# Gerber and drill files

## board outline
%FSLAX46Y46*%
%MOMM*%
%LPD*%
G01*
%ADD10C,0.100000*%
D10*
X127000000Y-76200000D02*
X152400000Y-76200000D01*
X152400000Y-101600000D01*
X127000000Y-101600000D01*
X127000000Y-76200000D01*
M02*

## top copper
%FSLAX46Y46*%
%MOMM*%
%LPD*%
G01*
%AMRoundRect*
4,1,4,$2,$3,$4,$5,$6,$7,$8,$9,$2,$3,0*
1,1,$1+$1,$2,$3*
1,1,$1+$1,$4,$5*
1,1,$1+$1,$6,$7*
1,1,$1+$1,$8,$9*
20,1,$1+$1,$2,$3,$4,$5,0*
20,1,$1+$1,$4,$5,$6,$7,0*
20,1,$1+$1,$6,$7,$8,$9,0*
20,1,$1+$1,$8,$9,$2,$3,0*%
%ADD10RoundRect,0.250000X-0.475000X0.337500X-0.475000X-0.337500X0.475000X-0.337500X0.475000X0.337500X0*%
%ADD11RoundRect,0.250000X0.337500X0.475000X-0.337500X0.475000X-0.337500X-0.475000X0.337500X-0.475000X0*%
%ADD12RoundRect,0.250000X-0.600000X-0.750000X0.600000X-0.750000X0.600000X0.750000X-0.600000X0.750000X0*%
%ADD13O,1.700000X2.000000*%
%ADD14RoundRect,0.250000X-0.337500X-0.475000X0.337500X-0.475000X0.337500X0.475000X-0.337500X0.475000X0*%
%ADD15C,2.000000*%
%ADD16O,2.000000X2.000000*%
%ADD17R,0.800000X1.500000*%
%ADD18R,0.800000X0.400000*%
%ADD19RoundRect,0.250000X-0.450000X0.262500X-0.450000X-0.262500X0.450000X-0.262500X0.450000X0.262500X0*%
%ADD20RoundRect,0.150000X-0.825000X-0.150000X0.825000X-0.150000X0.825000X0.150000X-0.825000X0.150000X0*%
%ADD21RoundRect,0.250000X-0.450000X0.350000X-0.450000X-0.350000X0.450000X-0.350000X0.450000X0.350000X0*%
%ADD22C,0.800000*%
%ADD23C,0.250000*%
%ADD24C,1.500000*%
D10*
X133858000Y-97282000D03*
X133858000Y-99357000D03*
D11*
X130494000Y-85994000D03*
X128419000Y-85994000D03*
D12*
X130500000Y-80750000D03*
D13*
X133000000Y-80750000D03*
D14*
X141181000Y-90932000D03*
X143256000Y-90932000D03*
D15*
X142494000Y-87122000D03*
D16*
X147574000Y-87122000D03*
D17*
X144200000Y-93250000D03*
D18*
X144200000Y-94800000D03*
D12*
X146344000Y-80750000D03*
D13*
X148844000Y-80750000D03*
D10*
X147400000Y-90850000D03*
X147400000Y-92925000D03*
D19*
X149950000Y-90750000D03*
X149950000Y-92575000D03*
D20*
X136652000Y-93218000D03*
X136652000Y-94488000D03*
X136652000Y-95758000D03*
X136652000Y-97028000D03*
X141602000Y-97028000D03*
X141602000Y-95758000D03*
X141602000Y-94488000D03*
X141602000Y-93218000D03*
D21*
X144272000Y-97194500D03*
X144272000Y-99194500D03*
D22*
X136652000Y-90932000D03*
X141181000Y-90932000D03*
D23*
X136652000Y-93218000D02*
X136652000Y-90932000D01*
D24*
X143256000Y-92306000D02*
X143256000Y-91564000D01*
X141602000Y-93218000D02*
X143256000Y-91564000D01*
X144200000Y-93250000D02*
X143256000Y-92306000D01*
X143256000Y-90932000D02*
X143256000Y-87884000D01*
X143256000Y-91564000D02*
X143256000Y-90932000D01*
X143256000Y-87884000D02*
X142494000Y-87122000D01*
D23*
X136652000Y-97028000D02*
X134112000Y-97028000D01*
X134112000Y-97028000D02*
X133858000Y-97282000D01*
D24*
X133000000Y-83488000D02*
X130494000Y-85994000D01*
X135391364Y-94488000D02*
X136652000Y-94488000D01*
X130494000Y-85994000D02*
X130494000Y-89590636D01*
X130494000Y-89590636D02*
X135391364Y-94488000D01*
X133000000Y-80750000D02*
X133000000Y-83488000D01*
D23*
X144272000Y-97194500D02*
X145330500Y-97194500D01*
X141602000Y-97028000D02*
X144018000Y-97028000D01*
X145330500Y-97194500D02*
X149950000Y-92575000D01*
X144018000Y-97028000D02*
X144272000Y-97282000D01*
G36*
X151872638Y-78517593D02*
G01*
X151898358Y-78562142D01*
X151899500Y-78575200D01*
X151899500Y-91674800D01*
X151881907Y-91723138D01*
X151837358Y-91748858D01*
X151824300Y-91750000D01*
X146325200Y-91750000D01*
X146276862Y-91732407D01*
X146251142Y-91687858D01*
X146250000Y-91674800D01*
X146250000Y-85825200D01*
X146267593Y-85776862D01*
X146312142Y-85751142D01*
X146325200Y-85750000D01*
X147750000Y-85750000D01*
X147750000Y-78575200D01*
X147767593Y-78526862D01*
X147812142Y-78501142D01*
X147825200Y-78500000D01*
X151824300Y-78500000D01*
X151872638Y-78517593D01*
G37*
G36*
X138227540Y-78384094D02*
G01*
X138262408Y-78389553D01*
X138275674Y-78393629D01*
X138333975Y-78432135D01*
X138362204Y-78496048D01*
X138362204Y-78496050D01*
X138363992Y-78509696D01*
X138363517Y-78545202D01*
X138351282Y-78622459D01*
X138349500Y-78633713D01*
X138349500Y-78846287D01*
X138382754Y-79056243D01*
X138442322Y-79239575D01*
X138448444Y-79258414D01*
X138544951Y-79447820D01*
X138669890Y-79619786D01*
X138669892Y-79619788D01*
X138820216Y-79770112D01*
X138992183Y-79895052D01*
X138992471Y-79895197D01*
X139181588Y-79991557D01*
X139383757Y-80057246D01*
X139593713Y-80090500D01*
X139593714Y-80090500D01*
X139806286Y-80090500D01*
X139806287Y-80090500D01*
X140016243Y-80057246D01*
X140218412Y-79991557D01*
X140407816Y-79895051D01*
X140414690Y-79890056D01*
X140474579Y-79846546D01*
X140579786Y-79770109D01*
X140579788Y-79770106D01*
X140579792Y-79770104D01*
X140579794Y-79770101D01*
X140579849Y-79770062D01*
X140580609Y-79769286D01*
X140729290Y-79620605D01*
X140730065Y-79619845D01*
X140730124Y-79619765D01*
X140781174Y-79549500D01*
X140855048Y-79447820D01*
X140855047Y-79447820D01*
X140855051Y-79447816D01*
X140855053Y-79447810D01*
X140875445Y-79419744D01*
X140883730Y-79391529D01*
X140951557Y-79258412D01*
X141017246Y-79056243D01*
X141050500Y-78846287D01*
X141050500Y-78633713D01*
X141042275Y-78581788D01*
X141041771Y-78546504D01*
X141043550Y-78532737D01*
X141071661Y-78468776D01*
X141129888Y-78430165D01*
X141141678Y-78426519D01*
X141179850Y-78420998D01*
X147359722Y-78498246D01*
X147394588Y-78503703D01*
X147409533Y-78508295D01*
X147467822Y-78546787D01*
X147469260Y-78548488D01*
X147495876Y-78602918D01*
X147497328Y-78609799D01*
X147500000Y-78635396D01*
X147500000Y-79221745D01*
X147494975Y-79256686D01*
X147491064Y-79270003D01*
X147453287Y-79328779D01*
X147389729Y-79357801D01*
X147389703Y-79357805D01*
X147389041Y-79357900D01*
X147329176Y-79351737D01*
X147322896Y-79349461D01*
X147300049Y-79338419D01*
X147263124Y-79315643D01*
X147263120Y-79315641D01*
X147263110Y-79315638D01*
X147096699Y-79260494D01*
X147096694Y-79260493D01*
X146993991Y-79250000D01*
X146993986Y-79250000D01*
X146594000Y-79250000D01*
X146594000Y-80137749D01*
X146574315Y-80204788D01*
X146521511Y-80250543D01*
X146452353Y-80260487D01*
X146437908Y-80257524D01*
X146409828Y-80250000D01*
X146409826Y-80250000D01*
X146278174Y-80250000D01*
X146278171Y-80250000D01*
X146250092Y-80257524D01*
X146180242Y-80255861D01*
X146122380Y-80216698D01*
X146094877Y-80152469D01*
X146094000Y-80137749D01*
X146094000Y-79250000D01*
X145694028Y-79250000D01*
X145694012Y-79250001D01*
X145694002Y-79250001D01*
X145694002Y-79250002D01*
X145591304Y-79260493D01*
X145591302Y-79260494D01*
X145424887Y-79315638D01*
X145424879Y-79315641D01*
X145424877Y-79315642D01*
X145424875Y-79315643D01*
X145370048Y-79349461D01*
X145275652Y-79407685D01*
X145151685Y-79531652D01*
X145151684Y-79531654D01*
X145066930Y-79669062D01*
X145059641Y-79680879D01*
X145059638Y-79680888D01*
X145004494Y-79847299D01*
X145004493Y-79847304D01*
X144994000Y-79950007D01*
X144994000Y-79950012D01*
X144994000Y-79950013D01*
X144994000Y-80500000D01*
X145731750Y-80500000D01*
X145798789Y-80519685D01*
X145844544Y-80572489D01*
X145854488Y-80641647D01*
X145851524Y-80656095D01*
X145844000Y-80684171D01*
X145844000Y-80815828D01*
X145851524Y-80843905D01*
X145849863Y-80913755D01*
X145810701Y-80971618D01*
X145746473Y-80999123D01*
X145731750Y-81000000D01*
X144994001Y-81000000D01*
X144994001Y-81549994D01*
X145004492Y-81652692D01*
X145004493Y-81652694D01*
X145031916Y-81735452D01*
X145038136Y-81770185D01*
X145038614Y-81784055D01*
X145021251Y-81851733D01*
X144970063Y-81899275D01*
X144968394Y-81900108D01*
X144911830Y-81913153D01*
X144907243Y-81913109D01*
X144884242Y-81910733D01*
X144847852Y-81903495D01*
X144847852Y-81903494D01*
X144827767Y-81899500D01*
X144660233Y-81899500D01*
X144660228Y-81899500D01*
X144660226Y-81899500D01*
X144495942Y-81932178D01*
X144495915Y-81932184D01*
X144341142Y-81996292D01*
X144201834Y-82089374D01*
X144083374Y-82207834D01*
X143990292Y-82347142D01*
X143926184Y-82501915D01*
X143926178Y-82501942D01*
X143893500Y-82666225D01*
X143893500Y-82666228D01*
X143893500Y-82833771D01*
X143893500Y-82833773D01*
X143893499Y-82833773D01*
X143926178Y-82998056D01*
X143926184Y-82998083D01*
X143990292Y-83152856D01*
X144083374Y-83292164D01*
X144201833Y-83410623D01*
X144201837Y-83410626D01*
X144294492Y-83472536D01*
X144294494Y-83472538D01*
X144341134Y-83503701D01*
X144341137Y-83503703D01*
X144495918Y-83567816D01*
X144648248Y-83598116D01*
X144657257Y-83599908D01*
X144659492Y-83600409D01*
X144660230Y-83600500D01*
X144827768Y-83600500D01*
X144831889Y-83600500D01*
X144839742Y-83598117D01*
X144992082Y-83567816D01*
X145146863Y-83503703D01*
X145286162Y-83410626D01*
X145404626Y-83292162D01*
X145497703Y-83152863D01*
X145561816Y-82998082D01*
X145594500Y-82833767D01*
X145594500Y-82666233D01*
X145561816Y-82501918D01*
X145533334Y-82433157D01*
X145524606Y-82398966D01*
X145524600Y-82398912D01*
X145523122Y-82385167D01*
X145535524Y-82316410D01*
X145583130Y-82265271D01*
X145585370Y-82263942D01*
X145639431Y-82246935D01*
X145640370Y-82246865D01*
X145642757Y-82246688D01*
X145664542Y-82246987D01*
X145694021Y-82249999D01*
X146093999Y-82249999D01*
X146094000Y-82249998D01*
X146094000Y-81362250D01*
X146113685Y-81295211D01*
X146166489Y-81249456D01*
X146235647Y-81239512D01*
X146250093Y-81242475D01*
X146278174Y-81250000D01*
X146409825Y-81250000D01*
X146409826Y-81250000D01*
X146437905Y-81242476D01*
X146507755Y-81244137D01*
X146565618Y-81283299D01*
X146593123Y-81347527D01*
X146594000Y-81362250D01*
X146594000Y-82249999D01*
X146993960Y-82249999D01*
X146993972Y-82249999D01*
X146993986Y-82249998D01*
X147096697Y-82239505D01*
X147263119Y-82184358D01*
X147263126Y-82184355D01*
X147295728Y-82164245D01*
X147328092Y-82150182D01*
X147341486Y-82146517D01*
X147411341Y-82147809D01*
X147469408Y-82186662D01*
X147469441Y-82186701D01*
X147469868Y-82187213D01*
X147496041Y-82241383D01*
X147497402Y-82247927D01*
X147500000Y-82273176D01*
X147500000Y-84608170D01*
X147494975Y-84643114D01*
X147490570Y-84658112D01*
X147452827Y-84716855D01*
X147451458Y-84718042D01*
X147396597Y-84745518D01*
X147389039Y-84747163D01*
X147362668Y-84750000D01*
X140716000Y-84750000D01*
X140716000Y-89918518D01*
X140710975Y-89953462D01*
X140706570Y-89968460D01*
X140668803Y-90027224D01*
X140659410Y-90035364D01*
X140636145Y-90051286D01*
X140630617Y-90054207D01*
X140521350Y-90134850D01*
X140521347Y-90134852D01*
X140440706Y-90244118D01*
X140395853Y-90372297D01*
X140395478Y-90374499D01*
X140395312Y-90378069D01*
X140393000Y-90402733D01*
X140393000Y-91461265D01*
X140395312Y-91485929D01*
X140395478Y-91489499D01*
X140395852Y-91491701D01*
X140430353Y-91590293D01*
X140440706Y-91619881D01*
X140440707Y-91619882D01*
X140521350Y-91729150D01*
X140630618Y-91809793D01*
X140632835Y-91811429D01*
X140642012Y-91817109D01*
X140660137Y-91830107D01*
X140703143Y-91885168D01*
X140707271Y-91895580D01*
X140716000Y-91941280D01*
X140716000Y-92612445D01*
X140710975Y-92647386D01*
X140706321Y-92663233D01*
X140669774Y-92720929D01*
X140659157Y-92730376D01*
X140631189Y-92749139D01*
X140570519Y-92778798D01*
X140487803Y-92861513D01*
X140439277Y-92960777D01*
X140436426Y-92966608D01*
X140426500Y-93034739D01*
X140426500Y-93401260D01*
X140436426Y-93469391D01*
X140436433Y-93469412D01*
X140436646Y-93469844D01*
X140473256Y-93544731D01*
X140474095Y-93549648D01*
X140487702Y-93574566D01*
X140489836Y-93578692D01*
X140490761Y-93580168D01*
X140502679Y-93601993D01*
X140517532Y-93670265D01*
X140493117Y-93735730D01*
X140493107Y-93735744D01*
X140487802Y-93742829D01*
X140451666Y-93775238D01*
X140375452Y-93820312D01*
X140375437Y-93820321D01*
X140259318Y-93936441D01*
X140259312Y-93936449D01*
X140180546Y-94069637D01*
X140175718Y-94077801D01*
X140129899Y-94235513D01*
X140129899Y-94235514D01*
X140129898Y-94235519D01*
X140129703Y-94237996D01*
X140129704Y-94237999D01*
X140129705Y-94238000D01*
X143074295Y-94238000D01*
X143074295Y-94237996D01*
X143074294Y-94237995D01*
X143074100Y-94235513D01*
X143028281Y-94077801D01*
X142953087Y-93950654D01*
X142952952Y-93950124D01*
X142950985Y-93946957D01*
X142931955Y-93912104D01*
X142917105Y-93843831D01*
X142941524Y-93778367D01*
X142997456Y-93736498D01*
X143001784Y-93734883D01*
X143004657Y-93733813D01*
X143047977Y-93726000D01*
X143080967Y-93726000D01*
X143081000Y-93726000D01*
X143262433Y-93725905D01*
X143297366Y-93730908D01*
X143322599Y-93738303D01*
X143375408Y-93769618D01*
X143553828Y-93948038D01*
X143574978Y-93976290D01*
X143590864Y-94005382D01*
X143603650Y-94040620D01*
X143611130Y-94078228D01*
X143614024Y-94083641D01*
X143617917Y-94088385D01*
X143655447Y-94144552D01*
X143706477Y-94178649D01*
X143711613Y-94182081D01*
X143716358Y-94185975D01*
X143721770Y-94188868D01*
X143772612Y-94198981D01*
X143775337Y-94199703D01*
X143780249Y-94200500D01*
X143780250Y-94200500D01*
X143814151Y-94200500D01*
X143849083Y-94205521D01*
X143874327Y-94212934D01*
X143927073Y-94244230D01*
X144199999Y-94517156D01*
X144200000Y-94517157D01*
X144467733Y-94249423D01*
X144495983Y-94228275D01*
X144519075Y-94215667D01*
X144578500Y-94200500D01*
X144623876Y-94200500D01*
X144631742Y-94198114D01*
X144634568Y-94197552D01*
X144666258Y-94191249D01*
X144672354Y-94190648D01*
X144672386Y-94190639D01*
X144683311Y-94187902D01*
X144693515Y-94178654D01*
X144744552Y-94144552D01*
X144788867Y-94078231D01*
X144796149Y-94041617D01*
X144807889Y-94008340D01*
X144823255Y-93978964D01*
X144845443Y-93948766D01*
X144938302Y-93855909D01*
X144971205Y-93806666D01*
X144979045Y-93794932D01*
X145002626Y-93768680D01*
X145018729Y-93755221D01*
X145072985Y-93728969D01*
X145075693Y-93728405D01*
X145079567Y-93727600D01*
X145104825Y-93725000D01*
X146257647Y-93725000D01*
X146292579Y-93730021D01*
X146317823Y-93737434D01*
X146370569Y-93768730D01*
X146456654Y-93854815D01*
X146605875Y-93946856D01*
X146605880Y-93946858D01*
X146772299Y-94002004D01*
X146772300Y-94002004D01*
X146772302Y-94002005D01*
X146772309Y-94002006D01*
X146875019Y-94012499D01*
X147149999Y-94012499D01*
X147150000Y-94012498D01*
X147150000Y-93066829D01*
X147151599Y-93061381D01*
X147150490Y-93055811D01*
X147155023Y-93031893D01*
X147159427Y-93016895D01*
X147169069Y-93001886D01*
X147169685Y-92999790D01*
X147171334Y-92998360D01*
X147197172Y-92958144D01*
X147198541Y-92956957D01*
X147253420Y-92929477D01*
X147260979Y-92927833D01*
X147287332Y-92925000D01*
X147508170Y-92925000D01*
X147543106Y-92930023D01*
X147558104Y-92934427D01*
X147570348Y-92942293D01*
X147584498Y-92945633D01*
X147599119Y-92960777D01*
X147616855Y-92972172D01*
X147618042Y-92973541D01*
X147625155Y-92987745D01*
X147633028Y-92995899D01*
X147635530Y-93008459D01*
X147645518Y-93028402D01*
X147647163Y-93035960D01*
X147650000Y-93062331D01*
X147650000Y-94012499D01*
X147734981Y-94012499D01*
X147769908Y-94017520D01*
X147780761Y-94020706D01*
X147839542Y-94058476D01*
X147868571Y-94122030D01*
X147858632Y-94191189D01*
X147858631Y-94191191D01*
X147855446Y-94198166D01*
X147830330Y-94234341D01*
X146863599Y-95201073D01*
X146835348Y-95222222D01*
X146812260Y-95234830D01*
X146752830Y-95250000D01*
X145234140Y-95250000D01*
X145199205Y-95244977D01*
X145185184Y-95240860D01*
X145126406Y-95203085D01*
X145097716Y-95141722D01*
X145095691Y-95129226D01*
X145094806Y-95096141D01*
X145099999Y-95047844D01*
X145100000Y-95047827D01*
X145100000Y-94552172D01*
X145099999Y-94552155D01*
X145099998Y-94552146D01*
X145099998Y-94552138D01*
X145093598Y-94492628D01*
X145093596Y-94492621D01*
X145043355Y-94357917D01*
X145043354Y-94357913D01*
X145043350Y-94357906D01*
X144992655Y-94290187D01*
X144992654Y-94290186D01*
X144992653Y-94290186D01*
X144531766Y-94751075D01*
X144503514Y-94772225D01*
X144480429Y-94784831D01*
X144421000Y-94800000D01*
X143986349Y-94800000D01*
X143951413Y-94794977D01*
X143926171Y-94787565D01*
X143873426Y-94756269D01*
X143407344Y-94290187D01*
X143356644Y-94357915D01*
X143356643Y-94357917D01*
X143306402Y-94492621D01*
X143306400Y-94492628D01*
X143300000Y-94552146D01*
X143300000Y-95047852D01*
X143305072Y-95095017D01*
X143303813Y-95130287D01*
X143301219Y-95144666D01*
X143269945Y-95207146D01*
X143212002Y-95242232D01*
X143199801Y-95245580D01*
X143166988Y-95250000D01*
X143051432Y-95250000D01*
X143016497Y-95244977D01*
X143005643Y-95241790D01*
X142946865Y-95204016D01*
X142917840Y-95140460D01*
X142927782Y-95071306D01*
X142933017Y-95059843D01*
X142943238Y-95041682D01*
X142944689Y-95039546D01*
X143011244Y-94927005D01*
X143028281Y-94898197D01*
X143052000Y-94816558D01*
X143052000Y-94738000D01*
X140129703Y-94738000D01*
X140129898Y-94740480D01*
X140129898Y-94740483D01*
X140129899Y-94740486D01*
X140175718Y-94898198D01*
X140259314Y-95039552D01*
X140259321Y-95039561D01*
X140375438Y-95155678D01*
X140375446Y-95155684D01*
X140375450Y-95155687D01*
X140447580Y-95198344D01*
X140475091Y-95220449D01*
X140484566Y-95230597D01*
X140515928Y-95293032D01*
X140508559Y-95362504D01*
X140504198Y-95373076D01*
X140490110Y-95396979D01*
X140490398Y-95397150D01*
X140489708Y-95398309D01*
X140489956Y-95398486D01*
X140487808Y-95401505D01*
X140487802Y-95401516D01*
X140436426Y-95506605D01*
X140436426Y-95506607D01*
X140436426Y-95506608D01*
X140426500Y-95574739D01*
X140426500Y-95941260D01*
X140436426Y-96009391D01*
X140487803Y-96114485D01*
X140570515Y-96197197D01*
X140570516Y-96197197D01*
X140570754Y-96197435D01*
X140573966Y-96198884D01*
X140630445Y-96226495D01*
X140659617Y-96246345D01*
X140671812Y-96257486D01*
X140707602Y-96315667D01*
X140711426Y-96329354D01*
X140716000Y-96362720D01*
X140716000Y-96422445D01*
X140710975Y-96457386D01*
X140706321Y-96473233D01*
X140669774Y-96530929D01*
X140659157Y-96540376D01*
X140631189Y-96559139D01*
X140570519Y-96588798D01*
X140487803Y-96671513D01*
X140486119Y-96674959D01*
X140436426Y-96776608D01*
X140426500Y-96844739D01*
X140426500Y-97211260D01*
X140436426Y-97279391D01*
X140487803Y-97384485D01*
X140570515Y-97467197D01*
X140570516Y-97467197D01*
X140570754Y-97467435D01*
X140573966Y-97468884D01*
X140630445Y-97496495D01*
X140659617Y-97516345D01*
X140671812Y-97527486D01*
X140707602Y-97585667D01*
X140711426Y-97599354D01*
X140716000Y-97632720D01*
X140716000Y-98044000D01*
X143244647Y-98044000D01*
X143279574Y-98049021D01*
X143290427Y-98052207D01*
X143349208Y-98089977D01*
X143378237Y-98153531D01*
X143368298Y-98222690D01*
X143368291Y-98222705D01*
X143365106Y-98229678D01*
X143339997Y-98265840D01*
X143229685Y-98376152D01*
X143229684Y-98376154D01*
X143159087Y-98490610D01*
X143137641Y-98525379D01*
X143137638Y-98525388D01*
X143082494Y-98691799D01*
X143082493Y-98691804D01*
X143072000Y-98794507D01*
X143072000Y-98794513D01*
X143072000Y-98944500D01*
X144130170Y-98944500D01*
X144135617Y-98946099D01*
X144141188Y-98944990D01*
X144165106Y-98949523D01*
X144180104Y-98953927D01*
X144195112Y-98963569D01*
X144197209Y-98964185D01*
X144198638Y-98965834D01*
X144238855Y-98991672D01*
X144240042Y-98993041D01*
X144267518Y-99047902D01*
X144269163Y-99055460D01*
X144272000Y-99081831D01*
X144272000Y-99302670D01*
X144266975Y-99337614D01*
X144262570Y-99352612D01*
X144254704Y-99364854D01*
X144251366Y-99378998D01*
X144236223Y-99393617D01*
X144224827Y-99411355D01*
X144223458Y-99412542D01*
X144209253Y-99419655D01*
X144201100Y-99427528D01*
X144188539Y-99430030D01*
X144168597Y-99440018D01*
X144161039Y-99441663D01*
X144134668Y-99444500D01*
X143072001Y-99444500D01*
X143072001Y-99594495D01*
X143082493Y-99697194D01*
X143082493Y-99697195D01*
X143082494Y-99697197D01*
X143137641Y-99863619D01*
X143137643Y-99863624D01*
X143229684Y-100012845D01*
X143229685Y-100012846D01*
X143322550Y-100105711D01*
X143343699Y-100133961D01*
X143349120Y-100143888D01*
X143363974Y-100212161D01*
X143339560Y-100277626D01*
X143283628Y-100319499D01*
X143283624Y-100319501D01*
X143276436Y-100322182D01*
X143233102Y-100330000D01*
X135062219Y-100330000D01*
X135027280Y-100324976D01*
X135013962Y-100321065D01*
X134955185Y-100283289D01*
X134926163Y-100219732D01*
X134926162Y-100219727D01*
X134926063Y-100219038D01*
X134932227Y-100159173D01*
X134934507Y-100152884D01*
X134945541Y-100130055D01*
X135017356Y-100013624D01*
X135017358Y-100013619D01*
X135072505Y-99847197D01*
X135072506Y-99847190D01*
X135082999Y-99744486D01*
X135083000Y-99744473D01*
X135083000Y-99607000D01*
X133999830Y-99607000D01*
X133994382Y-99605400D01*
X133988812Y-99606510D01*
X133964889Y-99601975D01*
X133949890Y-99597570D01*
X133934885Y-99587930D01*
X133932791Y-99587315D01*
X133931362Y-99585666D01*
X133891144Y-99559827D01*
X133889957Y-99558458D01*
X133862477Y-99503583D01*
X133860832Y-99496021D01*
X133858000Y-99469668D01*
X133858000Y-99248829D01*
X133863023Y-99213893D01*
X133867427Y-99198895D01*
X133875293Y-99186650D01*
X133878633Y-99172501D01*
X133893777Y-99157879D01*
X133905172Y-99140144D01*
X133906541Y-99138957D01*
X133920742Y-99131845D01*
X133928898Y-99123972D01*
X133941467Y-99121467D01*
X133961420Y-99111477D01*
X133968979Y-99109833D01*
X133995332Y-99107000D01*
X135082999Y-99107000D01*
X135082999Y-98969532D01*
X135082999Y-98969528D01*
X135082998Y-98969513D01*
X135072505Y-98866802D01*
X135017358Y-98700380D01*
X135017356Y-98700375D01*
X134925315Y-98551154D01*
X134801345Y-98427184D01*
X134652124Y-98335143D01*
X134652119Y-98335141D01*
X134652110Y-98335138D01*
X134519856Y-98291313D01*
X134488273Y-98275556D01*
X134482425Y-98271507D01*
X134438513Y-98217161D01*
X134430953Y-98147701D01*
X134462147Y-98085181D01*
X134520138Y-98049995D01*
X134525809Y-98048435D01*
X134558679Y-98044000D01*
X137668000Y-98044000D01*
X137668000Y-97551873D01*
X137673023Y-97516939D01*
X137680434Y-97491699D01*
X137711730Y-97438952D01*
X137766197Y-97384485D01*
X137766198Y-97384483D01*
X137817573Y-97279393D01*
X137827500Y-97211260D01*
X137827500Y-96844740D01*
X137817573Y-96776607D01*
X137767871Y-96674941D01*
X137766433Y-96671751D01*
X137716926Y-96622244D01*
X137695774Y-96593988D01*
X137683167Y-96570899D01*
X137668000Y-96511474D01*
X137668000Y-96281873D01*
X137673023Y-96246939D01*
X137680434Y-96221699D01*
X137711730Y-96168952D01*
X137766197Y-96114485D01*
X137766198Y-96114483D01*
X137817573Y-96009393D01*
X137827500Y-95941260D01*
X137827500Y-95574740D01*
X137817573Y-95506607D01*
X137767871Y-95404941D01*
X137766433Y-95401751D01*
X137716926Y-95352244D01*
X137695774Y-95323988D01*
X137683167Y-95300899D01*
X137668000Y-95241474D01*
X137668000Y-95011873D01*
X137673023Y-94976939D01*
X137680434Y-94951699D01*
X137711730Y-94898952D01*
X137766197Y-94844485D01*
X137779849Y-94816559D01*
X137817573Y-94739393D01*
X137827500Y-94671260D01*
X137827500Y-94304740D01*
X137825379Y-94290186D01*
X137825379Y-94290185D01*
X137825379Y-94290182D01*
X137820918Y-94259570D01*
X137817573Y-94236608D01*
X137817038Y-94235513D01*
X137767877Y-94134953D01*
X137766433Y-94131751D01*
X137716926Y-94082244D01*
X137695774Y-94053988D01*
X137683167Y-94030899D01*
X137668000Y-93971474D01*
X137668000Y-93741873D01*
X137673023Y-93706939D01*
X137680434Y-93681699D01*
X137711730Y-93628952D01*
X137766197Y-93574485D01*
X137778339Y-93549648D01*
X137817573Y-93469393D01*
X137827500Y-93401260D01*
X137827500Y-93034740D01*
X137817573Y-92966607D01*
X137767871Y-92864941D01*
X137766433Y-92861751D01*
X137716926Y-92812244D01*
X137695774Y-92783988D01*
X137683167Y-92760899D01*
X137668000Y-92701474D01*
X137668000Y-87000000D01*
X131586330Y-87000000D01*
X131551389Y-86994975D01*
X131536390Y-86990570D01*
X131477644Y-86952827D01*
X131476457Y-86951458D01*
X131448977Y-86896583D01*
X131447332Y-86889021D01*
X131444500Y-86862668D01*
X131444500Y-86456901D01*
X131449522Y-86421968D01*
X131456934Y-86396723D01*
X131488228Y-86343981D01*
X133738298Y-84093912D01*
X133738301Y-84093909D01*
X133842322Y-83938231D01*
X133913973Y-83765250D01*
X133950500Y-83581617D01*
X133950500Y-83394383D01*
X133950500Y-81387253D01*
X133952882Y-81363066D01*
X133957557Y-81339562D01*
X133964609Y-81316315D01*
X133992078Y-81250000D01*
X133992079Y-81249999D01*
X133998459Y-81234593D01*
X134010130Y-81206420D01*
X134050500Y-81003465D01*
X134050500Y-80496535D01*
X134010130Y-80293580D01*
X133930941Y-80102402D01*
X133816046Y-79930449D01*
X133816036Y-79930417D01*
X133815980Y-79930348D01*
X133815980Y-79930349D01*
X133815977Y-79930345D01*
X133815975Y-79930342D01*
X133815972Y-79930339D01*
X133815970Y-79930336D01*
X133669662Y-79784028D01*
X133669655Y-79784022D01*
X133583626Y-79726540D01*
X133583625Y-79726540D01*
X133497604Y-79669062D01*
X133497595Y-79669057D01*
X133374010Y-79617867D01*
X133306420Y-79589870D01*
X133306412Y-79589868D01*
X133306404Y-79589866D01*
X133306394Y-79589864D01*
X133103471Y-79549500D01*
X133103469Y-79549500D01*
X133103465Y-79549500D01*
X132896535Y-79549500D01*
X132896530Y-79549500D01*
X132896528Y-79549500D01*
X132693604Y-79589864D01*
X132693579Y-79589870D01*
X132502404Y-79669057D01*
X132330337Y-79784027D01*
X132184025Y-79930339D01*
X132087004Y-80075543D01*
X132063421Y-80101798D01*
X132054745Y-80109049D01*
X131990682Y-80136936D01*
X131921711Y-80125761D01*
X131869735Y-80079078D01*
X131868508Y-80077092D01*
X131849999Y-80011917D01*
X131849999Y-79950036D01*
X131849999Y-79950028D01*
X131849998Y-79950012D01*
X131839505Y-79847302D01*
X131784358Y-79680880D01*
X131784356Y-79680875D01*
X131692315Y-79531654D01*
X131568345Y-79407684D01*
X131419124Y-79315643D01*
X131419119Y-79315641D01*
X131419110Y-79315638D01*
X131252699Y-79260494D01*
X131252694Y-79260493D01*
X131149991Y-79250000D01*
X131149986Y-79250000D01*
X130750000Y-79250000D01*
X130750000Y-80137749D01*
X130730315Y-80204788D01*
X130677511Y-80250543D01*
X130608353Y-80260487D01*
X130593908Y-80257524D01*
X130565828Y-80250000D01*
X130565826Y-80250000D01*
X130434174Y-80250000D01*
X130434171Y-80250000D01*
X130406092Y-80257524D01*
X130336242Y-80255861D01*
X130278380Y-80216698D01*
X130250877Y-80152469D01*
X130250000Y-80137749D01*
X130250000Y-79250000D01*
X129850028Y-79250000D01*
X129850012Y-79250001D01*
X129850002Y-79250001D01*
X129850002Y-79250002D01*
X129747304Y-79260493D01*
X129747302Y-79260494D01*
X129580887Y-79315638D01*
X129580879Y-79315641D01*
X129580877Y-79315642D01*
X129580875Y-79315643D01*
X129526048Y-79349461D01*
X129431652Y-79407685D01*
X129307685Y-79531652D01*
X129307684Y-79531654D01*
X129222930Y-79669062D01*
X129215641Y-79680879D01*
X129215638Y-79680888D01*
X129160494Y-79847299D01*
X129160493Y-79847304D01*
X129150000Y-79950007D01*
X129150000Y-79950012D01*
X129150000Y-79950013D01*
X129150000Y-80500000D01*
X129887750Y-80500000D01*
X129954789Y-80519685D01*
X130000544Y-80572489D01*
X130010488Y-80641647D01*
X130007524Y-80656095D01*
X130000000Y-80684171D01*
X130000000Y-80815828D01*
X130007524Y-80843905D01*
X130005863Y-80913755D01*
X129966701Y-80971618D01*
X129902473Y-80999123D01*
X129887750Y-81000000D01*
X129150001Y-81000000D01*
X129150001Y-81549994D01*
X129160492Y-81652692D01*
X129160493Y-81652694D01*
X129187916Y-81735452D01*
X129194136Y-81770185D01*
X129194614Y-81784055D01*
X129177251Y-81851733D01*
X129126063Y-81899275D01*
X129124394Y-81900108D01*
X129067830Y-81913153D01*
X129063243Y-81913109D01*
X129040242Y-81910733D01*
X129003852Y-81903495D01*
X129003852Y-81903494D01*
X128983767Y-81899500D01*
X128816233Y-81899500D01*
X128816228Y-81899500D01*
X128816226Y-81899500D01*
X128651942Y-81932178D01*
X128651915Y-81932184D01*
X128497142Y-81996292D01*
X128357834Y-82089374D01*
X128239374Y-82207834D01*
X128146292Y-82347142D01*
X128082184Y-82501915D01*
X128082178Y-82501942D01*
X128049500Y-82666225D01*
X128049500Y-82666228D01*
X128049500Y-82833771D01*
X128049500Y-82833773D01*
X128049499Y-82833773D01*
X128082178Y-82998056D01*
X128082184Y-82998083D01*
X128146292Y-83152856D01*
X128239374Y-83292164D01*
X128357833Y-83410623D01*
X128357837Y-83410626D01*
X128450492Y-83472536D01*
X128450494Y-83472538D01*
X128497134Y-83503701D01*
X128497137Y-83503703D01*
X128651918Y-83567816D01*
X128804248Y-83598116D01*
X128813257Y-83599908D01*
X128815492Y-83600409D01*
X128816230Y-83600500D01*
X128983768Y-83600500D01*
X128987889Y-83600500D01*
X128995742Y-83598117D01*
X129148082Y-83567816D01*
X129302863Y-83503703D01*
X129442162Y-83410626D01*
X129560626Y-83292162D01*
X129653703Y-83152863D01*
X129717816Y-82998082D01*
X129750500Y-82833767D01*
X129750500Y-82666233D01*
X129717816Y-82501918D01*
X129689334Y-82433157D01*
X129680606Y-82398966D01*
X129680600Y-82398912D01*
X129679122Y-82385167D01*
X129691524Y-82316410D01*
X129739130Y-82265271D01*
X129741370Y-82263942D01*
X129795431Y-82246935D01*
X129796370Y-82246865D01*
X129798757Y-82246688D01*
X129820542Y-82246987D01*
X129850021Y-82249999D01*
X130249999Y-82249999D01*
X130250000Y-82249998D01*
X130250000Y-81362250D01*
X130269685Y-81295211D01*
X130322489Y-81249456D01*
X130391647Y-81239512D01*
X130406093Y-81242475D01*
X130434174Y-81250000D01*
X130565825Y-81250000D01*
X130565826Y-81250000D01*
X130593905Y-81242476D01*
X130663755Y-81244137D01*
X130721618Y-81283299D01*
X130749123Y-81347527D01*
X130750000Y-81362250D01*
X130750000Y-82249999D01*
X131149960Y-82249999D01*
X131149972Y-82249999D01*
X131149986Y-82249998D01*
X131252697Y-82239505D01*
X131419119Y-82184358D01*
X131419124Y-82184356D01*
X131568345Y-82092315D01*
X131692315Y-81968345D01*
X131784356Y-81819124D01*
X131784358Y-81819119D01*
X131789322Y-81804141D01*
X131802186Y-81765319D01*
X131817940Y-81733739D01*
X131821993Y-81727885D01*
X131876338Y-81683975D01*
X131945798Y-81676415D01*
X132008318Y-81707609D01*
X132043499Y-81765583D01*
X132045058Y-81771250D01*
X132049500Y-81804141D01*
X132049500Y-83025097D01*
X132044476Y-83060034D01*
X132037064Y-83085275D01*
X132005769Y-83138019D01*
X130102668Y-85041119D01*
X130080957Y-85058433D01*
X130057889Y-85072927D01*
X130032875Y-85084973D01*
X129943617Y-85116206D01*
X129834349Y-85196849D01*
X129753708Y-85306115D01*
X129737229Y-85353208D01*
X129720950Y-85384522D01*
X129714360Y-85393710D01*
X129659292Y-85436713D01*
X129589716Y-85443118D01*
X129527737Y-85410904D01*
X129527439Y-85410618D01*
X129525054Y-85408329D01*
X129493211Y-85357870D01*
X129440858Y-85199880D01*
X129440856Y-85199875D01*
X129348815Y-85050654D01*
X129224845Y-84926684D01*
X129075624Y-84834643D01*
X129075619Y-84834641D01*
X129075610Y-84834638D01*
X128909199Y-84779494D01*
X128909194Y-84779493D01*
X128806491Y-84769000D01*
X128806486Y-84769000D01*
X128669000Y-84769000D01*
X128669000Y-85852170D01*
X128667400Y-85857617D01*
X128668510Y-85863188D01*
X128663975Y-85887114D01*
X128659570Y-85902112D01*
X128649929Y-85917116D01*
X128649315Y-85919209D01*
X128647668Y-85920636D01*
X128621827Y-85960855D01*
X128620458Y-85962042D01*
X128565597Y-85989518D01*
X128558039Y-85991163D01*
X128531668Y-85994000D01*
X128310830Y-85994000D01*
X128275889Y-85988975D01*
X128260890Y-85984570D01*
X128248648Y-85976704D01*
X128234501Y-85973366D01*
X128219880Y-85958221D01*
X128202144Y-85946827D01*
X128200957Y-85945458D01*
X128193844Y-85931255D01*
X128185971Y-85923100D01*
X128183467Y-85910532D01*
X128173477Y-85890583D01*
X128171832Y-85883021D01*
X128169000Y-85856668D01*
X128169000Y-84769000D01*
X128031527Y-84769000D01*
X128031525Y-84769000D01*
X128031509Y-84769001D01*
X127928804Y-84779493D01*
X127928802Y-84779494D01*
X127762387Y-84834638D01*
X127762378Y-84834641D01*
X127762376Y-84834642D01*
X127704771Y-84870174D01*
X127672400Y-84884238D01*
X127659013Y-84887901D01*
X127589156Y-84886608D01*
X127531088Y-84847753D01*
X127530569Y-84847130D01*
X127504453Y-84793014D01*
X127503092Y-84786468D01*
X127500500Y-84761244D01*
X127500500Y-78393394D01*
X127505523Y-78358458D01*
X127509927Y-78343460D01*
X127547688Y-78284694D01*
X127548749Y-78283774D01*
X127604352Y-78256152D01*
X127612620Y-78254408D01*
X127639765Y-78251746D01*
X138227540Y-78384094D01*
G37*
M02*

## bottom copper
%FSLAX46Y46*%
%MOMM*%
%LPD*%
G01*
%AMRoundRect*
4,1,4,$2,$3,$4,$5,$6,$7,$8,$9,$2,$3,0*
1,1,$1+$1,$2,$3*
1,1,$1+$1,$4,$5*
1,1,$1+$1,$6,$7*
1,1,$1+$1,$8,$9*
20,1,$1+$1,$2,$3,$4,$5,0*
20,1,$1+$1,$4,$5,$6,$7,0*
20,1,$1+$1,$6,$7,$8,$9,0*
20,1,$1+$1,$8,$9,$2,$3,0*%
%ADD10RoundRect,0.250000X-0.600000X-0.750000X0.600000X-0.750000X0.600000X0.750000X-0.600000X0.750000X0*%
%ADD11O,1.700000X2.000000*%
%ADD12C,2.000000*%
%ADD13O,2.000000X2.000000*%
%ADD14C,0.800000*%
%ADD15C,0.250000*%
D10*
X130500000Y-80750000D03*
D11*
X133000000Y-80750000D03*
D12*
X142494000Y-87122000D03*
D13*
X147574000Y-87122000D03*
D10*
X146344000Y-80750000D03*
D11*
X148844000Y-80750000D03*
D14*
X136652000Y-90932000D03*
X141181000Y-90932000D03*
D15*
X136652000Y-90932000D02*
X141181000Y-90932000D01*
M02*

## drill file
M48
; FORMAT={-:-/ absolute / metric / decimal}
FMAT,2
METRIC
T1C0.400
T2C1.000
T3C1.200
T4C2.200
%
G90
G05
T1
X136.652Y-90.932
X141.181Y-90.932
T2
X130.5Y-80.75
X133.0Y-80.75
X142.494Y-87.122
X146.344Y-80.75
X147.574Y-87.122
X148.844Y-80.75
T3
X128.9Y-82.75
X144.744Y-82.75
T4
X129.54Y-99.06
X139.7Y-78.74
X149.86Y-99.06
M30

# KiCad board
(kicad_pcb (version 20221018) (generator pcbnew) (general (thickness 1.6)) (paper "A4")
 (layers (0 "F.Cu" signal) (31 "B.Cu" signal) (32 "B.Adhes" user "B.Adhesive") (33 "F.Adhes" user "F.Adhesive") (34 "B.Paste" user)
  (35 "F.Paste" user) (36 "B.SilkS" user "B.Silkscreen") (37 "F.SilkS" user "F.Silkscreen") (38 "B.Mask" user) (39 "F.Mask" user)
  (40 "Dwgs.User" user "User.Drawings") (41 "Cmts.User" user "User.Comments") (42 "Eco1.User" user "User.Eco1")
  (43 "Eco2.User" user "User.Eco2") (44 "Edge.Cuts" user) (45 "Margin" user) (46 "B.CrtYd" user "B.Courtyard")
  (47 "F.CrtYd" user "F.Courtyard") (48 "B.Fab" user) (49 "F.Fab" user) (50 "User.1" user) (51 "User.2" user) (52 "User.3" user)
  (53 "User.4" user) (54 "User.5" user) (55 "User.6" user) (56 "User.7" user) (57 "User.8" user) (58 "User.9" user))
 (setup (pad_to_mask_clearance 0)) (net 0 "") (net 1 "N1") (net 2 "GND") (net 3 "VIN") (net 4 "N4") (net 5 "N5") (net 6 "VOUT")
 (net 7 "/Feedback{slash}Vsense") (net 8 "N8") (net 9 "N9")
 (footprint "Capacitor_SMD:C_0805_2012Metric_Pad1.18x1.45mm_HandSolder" (layer "F.Cu") (at 133.858 98.3195 -90)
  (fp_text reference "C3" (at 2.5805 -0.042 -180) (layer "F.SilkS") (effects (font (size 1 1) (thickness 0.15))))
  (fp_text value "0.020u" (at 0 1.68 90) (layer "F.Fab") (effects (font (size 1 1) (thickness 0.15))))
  (pad "1" smd roundrect (at -1.0375 0 270) (size 1.175 1.45) (layers "F.Cu" "F.Paste" "F.Mask") (roundrect_rratio 0.212766) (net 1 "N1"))
  (pad "2" smd roundrect (at 1.0375 0 270) (size 1.175 1.45) (layers "F.Cu" "F.Paste" "F.Mask") (roundrect_rratio 0.212766) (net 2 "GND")))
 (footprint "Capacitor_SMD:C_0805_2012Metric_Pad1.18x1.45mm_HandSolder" (layer "F.Cu") (at 129.4565 85.994 180)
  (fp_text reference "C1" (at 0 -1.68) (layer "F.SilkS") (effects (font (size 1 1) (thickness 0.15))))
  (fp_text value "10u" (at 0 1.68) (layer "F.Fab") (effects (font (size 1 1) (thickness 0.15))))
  (pad "1" smd roundrect (at -1.0375 0 180) (size 1.175 1.45) (layers "F.Cu" "F.Paste" "F.Mask") (roundrect_rratio 0.212766) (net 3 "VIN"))
  (pad "2" smd roundrect (at 1.0375 0 180) (size 1.175 1.45) (layers "F.Cu" "F.Paste" "F.Mask") (roundrect_rratio 0.212766) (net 2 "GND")))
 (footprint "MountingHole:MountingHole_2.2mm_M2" (layer "F.Cu") (at 139.7 78.74)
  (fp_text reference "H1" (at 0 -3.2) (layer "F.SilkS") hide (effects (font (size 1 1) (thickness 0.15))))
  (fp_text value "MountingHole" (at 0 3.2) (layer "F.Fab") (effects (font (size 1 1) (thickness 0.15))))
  (pad "" np_thru_hole circle (at 0 0) (size 2.2 2.2) (drill 2.2) (layers "*.Cu" "*.Mask")))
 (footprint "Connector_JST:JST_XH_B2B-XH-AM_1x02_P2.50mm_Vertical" (layer "F.Cu") (at 130.5 80.75)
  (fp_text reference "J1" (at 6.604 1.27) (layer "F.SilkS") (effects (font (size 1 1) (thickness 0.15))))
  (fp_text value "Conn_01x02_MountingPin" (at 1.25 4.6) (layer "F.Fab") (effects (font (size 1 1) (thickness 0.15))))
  (pad "" np_thru_hole circle (at -1.6 2) (size 1.2 1.2) (drill 1.2) (layers "*.Cu" "*.Mask"))
  (pad "1" thru_hole roundrect (at 0 0) (size 1.7 2) (drill 1) (layers "*.Cu" "*.Mask") (roundrect_rratio 0.147059) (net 2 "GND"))
  (pad "2" thru_hole oval (at 2.5 0) (size 1.7 2) (drill 1) (layers "*.Cu" "*.Mask") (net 3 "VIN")))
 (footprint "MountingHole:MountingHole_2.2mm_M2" (layer "F.Cu") (at 129.54 99.06)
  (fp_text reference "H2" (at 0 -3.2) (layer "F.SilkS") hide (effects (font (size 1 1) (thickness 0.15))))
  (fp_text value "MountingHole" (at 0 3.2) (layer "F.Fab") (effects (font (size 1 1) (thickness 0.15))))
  (pad "" np_thru_hole circle (at 0 0) (size 2.2 2.2) (drill 2.2) (layers "*.Cu" "*.Mask")))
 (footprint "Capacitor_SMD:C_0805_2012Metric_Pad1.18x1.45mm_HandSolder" (layer "F.Cu") (at 142.2185 90.932)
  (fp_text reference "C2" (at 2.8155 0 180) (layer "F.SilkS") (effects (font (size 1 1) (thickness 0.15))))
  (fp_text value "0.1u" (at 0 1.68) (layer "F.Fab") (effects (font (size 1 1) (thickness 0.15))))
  (pad "1" smd roundrect (at -1.0375 0) (size 1.175 1.45) (layers "F.Cu" "F.Paste" "F.Mask") (roundrect_rratio 0.212766) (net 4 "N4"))
  (pad "2" smd roundrect (at 1.0375 0) (size 1.175 1.45) (layers "F.Cu" "F.Paste" "F.Mask") (roundrect_rratio 0.212766) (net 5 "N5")))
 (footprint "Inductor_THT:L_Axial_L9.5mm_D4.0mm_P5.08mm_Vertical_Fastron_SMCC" (layer "F.Cu") (at 142.494 87.122)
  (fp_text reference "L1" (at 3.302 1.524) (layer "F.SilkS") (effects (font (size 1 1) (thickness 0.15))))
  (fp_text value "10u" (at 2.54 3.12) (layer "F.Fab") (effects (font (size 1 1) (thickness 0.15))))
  (pad "1" thru_hole circle (at 0 0) (size 2 2) (drill 1) (layers "*.Cu" "*.Mask") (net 5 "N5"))
  (pad "2" thru_hole oval (at 5.08 0) (size 2 2) (drill 1) (layers "*.Cu" "*.Mask") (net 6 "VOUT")))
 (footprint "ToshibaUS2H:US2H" (layer "F.Cu") (at 144.2 94 -90)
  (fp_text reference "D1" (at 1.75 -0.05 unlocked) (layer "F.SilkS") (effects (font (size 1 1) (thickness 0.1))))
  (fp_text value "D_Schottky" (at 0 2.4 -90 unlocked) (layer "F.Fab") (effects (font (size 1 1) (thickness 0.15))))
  (pad "1" smd rect (at -0.75 0) (size 0.8 1.5) (layers "F.Cu" "F.Paste" "F.Mask") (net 5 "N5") (thermal_bridge_angle 45))
  (pad "2" smd rect (at 0.8 0) (size 0.8 0.4) (layers "F.Cu" "F.Paste" "F.Mask") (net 2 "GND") (thermal_bridge_angle 45)))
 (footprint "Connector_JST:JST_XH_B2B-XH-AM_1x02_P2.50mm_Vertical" (layer "F.Cu") (at 146.344 80.75)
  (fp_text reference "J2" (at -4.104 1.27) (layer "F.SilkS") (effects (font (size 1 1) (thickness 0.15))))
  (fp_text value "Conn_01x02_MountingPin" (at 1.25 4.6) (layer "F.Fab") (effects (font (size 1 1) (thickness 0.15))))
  (pad "" np_thru_hole circle (at -1.6 2) (size 1.2 1.2) (drill 1.2) (layers "*.Cu" "*.Mask"))
  (pad "1" thru_hole roundrect (at 0 0) (size 1.7 2) (drill 1) (layers "*.Cu" "*.Mask") (roundrect_rratio 0.147059) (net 2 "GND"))
  (pad "2" thru_hole oval (at 2.5 0) (size 1.7 2) (drill 1) (layers "*.Cu" "*.Mask") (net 6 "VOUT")))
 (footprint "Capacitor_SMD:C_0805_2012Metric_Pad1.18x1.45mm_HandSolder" (layer "F.Cu") (at 147.4 91.8875 -90)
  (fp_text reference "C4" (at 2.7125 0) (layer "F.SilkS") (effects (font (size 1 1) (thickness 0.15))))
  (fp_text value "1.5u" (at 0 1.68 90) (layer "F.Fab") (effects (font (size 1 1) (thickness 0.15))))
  (pad "1" smd roundrect (at -1.0375 0 270) (size 1.175 1.45) (layers "F.Cu" "F.Paste" "F.Mask") (roundrect_rratio 0.212766) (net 6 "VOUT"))
  (pad "2" smd roundrect (at 1.0375 0 270) (size 1.175 1.45) (layers "F.Cu" "F.Paste" "F.Mask") (roundrect_rratio 0.212766) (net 2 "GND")))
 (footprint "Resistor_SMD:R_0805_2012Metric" (layer "F.Cu") (at 149.95 91.6625 -90)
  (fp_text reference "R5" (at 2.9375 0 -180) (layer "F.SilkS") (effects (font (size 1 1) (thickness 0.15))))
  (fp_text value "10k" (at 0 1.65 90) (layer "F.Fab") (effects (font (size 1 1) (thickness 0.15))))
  (pad "1" smd roundrect (at -0.9125 0 270) (size 1.025 1.4) (layers "F.Cu" "F.Paste" "F.Mask") (roundrect_rratio 0.243902) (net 6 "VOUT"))
  (pad "2" smd roundrect (at 0.9125 0 270) (size 1.025 1.4) (layers "F.Cu" "F.Paste" "F.Mask") (roundrect_rratio 0.243902)
   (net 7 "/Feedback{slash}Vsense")))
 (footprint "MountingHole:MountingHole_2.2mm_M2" (layer "F.Cu") (at 149.86 99.06)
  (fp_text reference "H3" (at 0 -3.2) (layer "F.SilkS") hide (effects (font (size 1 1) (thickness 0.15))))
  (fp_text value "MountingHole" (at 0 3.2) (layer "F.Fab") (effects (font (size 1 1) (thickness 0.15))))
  (pad "" np_thru_hole circle (at 0 0) (size 2.2 2.2) (drill 2.2) (layers "*.Cu" "*.Mask")))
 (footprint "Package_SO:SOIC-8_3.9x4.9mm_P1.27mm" (layer "F.Cu") (at 139.127 95.123)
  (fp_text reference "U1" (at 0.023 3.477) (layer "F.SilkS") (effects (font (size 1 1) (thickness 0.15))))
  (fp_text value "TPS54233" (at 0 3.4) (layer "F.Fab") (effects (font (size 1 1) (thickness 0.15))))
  (pad "1" smd roundrect (at -2.475 -1.905) (size 1.95 0.6) (layers "F.Cu" "F.Paste" "F.Mask") (roundrect_rratio 0.25) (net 4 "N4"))
  (pad "2" smd roundrect (at -2.475 -0.635) (size 1.95 0.6) (layers "F.Cu" "F.Paste" "F.Mask") (roundrect_rratio 0.25) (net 3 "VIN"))
  (pad "3" smd roundrect (at -2.475 0.635) (size 1.95 0.6) (layers "F.Cu" "F.Paste" "F.Mask") (roundrect_rratio 0.25) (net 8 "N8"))
  (pad "4" smd roundrect (at -2.475 1.905) (size 1.95 0.6) (layers "F.Cu" "F.Paste" "F.Mask") (roundrect_rratio 0.25) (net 1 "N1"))
  (pad "5" smd roundrect (at 2.475 1.905) (size 1.95 0.6) (layers "F.Cu" "F.Paste" "F.Mask") (roundrect_rratio 0.25)
   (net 7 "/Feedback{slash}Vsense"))
  (pad "6" smd roundrect (at 2.475 0.635) (size 1.95 0.6) (layers "F.Cu" "F.Paste" "F.Mask") (roundrect_rratio 0.25) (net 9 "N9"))
  (pad "7" smd roundrect (at 2.475 -0.635) (size 1.95 0.6) (layers "F.Cu" "F.Paste" "F.Mask") (roundrect_rratio 0.25) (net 2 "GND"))
  (pad "8" smd roundrect (at 2.475 -1.905) (size 1.95 0.6) (layers "F.Cu" "F.Paste" "F.Mask") (roundrect_rratio 0.25) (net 5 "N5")))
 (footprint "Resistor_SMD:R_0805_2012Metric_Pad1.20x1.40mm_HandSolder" (layer "F.Cu") (at 144.272 98.1945 -90)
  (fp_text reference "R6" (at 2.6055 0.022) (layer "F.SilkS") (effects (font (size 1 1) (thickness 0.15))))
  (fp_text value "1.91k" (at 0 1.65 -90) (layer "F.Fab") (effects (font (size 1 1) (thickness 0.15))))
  (pad "1" smd roundrect (at -1 0 270) (size 1.2 1.4) (layers "F.Cu" "F.Paste" "F.Mask") (roundrect_rratio 0.208333)
   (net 7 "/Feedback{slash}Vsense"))
  (pad "2" smd roundrect (at 1 0 270) (size 1.2 1.4) (layers "F.Cu" "F.Paste" "F.Mask") (roundrect_rratio 0.208333) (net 2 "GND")))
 (gr_rect (start 127 76.2) (end 152.4 101.6) (stroke (width 0.1) (type default)) (fill none) (layer "Edge.Cuts"))
 (segment (start 136.652 93.218) (end 136.652 90.932) (width 0.25) (layer "F.Cu") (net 4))
 (via (at 136.652 90.932) (size 0.8) (drill 0.4) (layers "F.Cu" "B.Cu") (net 4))
 (via (at 141.181 90.932) (size 0.8) (drill 0.4) (layers "F.Cu" "B.Cu") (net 4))
 (segment (start 136.652 90.932) (end 141.181 90.932) (width 0.25) (layer "B.Cu") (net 4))
 (segment (start 143.256 92.306) (end 143.256 91.564) (width 1.5) (layer "F.Cu") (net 5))
 (segment (start 141.602 93.218) (end 143.256 91.564) (width 1.5) (layer "F.Cu") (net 5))
 (segment (start 144.2 93.25) (end 143.256 92.306) (width 1.5) (layer "F.Cu") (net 5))
 (segment (start 143.256 90.932) (end 143.256 87.884) (width 1.5) (layer "F.Cu") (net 5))
 (segment (start 143.256 91.564) (end 143.256 90.932) (width 1.5) (layer "F.Cu") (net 5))
 (segment (start 143.256 87.884) (end 142.494 87.122) (width 1.5) (layer "F.Cu") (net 5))
 (segment (start 136.652 97.028) (end 134.112 97.028) (width 0.25) (layer "F.Cu") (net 1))
 (segment (start 134.112 97.028) (end 133.858 97.282) (width 0.25) (layer "F.Cu") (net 1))
 (segment (start 133 83.488) (end 130.494 85.994) (width 1.5) (layer "F.Cu") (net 3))
 (segment (start 135.391364 94.488) (end 136.652 94.488) (width 1.5) (layer "F.Cu") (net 3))
 (segment (start 130.494 85.994) (end 130.494 89.590636) (width 1.5) (layer "F.Cu") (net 3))
 (segment (start 130.494 89.590636) (end 135.391364 94.488) (width 1.5) (layer "F.Cu") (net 3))
 (segment (start 133 80.75) (end 133 83.488) (width 1.5) (layer "F.Cu") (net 3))
 (segment (start 144.272 97.1945) (end 145.3305 97.1945) (width 0.25) (layer "F.Cu") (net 7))
 (segment (start 141.602 97.028) (end 144.018 97.028) (width 0.25) (layer "F.Cu") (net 7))
 (segment (start 145.3305 97.1945) (end 149.95 92.575) (width 0.25) (layer "F.Cu") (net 7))
 (segment (start 144.018 97.028) (end 144.272 97.282) (width 0.25) (layer "F.Cu") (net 7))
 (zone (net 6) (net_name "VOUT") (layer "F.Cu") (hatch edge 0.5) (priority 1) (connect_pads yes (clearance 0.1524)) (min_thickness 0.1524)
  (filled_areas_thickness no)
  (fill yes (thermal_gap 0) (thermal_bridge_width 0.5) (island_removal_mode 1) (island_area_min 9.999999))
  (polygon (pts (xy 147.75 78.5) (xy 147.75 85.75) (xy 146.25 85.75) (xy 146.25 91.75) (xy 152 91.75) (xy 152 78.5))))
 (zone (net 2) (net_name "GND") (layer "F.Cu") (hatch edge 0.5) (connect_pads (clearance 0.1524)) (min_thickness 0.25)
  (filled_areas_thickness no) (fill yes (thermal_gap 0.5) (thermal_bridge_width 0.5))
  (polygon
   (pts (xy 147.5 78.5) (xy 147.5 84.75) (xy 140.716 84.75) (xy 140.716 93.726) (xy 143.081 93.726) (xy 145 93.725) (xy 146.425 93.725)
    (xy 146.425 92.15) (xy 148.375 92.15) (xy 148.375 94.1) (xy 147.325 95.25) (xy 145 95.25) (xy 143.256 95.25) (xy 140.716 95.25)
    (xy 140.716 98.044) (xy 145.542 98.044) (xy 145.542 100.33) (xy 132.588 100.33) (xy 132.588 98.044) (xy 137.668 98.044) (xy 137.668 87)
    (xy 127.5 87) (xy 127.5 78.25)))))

